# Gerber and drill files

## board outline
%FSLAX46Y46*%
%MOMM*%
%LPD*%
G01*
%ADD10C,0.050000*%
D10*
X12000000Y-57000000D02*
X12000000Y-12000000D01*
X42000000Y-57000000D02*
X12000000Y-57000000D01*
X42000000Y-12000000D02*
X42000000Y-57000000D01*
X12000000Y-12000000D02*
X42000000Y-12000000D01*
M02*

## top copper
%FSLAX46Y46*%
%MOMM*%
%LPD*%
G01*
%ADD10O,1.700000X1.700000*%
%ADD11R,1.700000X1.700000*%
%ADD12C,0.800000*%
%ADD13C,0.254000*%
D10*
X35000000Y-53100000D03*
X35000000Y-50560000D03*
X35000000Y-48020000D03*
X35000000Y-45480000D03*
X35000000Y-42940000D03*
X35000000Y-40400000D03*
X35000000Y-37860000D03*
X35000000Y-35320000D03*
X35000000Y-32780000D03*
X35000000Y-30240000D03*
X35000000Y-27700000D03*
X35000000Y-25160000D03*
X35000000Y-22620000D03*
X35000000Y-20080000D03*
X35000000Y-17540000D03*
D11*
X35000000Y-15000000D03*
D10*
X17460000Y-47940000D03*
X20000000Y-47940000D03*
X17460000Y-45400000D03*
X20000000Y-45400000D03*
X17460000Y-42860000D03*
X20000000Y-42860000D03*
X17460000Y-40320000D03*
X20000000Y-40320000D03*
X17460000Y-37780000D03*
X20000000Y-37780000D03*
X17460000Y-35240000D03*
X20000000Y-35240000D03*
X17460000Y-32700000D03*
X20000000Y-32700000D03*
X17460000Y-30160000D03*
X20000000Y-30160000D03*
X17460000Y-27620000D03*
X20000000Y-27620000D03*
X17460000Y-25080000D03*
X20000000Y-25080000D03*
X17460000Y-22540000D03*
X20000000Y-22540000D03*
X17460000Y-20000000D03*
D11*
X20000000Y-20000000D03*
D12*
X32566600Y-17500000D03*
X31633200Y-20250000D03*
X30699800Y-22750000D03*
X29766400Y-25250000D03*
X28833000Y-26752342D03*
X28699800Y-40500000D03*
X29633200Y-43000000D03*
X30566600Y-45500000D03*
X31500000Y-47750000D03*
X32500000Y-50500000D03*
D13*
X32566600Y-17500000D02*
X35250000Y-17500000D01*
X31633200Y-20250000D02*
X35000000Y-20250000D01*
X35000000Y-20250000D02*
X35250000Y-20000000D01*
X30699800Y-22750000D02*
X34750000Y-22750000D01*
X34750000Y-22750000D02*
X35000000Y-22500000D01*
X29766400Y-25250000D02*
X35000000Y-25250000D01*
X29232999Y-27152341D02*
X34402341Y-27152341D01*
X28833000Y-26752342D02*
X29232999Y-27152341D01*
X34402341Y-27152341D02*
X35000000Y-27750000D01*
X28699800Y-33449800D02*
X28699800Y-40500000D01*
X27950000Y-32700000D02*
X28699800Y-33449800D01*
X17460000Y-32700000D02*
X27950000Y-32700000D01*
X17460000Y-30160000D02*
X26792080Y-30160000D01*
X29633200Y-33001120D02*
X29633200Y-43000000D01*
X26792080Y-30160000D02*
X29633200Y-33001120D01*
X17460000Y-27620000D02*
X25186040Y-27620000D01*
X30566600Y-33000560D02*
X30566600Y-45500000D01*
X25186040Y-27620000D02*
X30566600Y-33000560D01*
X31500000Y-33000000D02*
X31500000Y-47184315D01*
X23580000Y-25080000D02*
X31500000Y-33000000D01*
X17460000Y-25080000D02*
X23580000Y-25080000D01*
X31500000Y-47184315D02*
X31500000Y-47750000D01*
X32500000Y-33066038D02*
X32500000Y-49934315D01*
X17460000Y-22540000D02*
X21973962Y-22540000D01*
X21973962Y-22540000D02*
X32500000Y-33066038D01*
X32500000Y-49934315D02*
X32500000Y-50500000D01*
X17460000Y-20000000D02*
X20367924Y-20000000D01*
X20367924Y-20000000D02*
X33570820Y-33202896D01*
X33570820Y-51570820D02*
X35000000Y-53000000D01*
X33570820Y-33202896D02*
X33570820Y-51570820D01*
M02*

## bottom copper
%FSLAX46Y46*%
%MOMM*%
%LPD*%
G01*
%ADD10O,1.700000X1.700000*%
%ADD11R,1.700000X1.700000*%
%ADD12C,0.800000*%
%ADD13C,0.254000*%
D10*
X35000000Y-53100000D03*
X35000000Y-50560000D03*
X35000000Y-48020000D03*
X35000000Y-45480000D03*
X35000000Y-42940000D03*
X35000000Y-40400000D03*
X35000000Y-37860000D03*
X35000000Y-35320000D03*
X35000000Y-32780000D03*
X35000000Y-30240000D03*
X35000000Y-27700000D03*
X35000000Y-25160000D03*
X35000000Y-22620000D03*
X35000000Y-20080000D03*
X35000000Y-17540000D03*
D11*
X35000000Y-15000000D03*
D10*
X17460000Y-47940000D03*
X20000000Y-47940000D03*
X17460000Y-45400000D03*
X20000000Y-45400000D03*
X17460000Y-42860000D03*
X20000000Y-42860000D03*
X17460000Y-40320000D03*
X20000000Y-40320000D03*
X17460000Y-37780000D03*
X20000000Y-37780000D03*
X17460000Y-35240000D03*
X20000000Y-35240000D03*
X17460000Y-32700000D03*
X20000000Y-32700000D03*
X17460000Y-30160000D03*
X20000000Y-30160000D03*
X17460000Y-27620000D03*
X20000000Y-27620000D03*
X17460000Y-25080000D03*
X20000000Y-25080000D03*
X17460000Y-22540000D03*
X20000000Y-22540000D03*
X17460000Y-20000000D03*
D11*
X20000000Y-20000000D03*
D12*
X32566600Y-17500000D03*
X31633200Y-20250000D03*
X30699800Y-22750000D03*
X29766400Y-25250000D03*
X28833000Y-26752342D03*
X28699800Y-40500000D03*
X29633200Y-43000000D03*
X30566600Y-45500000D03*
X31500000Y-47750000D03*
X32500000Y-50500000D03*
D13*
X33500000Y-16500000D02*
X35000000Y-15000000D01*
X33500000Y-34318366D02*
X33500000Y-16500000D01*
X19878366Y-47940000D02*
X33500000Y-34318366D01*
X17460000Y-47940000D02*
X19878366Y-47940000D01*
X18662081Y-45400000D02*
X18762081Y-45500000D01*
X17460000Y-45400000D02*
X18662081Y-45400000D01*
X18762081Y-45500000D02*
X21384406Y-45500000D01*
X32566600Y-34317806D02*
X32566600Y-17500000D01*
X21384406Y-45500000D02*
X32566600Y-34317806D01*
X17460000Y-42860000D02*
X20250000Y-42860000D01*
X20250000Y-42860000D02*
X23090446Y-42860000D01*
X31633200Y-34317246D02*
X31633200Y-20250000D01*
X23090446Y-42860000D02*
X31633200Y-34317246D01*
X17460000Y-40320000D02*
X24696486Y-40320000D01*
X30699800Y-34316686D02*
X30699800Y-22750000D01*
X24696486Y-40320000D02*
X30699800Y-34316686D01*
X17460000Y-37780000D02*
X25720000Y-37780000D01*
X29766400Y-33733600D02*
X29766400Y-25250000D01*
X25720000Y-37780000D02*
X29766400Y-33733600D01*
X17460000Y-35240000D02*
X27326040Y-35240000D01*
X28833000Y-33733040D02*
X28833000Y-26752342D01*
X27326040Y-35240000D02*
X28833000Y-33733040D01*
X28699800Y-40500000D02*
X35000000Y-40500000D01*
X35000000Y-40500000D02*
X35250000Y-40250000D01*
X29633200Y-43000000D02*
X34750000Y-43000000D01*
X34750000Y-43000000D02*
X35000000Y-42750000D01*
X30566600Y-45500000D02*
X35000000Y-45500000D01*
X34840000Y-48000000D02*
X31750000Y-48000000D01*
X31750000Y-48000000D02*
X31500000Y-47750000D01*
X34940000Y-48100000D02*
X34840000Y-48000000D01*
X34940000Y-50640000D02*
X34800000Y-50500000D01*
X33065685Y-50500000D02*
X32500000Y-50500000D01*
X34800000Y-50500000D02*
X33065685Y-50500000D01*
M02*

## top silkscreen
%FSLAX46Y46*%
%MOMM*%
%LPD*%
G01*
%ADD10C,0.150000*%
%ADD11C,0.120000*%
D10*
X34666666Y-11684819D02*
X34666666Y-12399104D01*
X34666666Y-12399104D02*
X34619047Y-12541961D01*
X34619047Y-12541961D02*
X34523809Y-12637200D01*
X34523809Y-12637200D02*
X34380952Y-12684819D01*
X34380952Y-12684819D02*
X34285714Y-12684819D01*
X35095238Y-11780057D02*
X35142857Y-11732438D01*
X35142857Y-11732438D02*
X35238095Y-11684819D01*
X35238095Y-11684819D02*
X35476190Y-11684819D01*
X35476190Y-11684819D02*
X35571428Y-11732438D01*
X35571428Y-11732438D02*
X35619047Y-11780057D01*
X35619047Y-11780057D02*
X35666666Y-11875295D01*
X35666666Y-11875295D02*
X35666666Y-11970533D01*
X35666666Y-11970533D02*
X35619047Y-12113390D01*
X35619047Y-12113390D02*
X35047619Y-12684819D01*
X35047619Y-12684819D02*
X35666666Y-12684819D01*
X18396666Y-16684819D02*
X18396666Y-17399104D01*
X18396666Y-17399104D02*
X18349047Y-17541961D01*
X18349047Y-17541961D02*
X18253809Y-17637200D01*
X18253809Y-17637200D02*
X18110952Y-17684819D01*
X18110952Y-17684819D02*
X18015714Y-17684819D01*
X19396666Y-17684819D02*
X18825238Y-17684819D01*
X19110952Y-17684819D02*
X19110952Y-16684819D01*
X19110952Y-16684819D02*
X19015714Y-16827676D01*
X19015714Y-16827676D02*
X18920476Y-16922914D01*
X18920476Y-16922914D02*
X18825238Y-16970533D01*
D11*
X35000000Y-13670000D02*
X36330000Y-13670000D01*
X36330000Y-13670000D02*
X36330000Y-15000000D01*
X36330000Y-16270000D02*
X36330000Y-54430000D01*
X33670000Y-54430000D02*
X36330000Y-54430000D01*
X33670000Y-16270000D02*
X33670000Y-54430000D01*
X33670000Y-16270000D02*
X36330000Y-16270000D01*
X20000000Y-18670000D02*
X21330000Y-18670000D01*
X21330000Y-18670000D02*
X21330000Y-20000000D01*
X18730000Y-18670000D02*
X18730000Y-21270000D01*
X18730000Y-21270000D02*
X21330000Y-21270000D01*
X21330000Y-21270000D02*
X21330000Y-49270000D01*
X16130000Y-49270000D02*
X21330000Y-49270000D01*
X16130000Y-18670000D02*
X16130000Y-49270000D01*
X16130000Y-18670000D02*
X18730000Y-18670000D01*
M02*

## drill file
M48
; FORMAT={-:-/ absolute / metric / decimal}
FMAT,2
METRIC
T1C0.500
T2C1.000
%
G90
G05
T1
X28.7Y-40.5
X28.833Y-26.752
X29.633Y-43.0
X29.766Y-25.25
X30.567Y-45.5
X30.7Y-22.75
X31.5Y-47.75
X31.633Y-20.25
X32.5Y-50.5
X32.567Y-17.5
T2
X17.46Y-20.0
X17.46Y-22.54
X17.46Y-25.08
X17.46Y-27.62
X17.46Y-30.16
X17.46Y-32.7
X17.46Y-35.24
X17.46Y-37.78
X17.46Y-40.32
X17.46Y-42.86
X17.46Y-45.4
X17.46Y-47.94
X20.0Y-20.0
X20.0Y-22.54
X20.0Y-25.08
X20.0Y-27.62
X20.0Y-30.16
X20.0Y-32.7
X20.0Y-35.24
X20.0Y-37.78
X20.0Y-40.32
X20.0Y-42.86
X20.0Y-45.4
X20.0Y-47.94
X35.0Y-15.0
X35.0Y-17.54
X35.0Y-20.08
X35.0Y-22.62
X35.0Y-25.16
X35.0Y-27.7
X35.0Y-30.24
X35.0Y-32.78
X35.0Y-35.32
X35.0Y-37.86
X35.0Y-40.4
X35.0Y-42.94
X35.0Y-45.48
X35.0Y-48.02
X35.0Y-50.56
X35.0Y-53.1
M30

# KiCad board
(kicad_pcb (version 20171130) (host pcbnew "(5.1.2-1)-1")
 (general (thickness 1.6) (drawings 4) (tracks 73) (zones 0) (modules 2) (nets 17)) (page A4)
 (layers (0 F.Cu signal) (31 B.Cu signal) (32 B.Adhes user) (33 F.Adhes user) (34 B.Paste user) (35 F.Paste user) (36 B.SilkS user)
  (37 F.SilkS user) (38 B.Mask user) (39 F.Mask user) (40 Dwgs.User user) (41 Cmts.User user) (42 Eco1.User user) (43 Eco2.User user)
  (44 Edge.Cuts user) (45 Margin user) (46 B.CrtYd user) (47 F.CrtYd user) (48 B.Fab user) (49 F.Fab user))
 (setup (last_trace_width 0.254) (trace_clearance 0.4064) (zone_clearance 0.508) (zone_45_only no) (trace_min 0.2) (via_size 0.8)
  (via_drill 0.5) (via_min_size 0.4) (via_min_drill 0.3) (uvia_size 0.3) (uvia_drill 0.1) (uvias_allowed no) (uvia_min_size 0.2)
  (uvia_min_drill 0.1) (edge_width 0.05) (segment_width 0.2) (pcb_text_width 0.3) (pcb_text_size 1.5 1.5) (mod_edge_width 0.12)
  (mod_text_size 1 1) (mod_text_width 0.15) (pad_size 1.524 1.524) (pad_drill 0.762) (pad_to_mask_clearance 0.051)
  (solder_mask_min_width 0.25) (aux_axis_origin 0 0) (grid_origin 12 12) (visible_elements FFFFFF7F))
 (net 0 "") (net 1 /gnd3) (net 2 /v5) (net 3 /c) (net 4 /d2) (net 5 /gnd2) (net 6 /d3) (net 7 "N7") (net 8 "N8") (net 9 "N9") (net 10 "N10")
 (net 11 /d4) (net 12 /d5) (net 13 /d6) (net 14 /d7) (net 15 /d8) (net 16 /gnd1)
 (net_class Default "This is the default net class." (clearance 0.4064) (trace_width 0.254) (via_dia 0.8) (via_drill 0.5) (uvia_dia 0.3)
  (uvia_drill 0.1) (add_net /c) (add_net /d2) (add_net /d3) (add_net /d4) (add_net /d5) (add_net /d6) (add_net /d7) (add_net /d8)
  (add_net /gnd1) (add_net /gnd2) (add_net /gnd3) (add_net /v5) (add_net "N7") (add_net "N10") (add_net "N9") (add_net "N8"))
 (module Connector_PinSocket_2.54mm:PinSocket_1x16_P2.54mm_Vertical (layer F.Cu) (at 35 15)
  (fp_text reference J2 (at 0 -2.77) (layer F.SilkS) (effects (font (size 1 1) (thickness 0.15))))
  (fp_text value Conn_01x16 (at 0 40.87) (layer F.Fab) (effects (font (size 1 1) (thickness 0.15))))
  (fp_line (start 0 -1.33) (end 1.33 -1.33) (layer F.SilkS) (width 0.12))
  (fp_line (start 1.33 -1.33) (end 1.33 0) (layer F.SilkS) (width 0.12))
  (fp_line (start 1.33 1.27) (end 1.33 39.43) (layer F.SilkS) (width 0.12))
  (fp_line (start -1.33 39.43) (end 1.33 39.43) (layer F.SilkS) (width 0.12))
  (fp_line (start -1.33 1.27) (end -1.33 39.43) (layer F.SilkS) (width 0.12))
  (fp_line (start -1.33 1.27) (end 1.33 1.27) (layer F.SilkS) (width 0.12))
  (pad 16 thru_hole oval (at 0 38.1) (size 1.7 1.7) (drill 1) (layers *.Cu *.Mask) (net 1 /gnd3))
  (pad 15 thru_hole oval (at 0 35.56) (size 1.7 1.7) (drill 1) (layers *.Cu *.Mask) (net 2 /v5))
  (pad 14 thru_hole oval (at 0 33.02) (size 1.7 1.7) (drill 1) (layers *.Cu *.Mask) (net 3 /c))
  (pad 13 thru_hole oval (at 0 30.48) (size 1.7 1.7) (drill 1) (layers *.Cu *.Mask) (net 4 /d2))
  (pad 12 thru_hole oval (at 0 27.94) (size 1.7 1.7) (drill 1) (layers *.Cu *.Mask) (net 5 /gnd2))
  (pad 11 thru_hole oval (at 0 25.4) (size 1.7 1.7) (drill 1) (layers *.Cu *.Mask) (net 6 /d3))
  (pad 10 thru_hole oval (at 0 22.86) (size 1.7 1.7) (drill 1) (layers *.Cu *.Mask) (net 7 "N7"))
  (pad 9 thru_hole oval (at 0 20.32) (size 1.7 1.7) (drill 1) (layers *.Cu *.Mask) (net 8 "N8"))
  (pad 8 thru_hole oval (at 0 17.78) (size 1.7 1.7) (drill 1) (layers *.Cu *.Mask) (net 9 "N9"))
  (pad 7 thru_hole oval (at 0 15.24) (size 1.7 1.7) (drill 1) (layers *.Cu *.Mask) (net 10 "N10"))
  (pad 6 thru_hole oval (at 0 12.7) (size 1.7 1.7) (drill 1) (layers *.Cu *.Mask) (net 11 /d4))
  (pad 5 thru_hole oval (at 0 10.16) (size 1.7 1.7) (drill 1) (layers *.Cu *.Mask) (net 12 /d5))
  (pad 4 thru_hole oval (at 0 7.62) (size 1.7 1.7) (drill 1) (layers *.Cu *.Mask) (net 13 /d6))
  (pad 3 thru_hole oval (at 0 5.08) (size 1.7 1.7) (drill 1) (layers *.Cu *.Mask) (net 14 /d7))
  (pad 2 thru_hole oval (at 0 2.54) (size 1.7 1.7) (drill 1) (layers *.Cu *.Mask) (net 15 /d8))
  (pad 1 thru_hole rect (at 0 0) (size 1.7 1.7) (drill 1) (layers *.Cu *.Mask) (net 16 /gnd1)))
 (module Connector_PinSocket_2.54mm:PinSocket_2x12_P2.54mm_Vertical (layer F.Cu) (at 20 20)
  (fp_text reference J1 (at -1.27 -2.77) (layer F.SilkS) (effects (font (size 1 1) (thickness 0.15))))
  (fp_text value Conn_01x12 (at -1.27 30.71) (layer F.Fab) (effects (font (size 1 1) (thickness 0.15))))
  (fp_line (start 0 -1.33) (end 1.33 -1.33) (layer F.SilkS) (width 0.12))
  (fp_line (start 1.33 -1.33) (end 1.33 0) (layer F.SilkS) (width 0.12))
  (fp_line (start -1.27 -1.33) (end -1.27 1.27) (layer F.SilkS) (width 0.12))
  (fp_line (start -1.27 1.27) (end 1.33 1.27) (layer F.SilkS) (width 0.12))
  (fp_line (start 1.33 1.27) (end 1.33 29.27) (layer F.SilkS) (width 0.12))
  (fp_line (start -3.87 29.27) (end 1.33 29.27) (layer F.SilkS) (width 0.12))
  (fp_line (start -3.87 -1.33) (end -3.87 29.27) (layer F.SilkS) (width 0.12))
  (fp_line (start -3.87 -1.33) (end -1.27 -1.33) (layer F.SilkS) (width 0.12))
  (pad 24 thru_hole oval (at -2.54 27.94) (size 1.7 1.7) (drill 1) (layers *.Cu *.Mask) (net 16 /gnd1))
  (pad 23 thru_hole oval (at 0 27.94) (size 1.7 1.7) (drill 1) (layers *.Cu *.Mask) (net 16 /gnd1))
  (pad 22 thru_hole oval (at -2.54 25.4) (size 1.7 1.7) (drill 1) (layers *.Cu *.Mask) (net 15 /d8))
  (pad 21 thru_hole oval (at 0 25.4) (size 1.7 1.7) (drill 1) (layers *.Cu *.Mask) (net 15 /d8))
  (pad 20 thru_hole oval (at -2.54 22.86) (size 1.7 1.7) (drill 1) (layers *.Cu *.Mask) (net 14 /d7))
  (pad 19 thru_hole oval (at 0 22.86) (size 1.7 1.7) (drill 1) (layers *.Cu *.Mask) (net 14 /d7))
  (pad 18 thru_hole oval (at -2.54 20.32) (size 1.7 1.7) (drill 1) (layers *.Cu *.Mask) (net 13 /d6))
  (pad 17 thru_hole oval (at 0 20.32) (size 1.7 1.7) (drill 1) (layers *.Cu *.Mask) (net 13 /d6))
  (pad 16 thru_hole oval (at -2.54 17.78) (size 1.7 1.7) (drill 1) (layers *.Cu *.Mask) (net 12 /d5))
  (pad 15 thru_hole oval (at 0 17.78) (size 1.7 1.7) (drill 1) (layers *.Cu *.Mask) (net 12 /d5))
  (pad 14 thru_hole oval (at -2.54 15.24) (size 1.7 1.7) (drill 1) (layers *.Cu *.Mask) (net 11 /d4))
  (pad 13 thru_hole oval (at 0 15.24) (size 1.7 1.7) (drill 1) (layers *.Cu *.Mask) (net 11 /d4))
  (pad 12 thru_hole oval (at -2.54 12.7) (size 1.7 1.7) (drill 1) (layers *.Cu *.Mask) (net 6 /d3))
  (pad 11 thru_hole oval (at 0 12.7) (size 1.7 1.7) (drill 1) (layers *.Cu *.Mask) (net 6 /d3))
  (pad 10 thru_hole oval (at -2.54 10.16) (size 1.7 1.7) (drill 1) (layers *.Cu *.Mask) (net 5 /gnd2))
  (pad 9 thru_hole oval (at 0 10.16) (size 1.7 1.7) (drill 1) (layers *.Cu *.Mask) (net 5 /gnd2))
  (pad 8 thru_hole oval (at -2.54 7.62) (size 1.7 1.7) (drill 1) (layers *.Cu *.Mask) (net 4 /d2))
  (pad 7 thru_hole oval (at 0 7.62) (size 1.7 1.7) (drill 1) (layers *.Cu *.Mask) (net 4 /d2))
  (pad 6 thru_hole oval (at -2.54 5.08) (size 1.7 1.7) (drill 1) (layers *.Cu *.Mask) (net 3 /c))
  (pad 5 thru_hole oval (at 0 5.08) (size 1.7 1.7) (drill 1) (layers *.Cu *.Mask) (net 3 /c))
  (pad 4 thru_hole oval (at -2.54 2.54) (size 1.7 1.7) (drill 1) (layers *.Cu *.Mask) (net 2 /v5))
  (pad 3 thru_hole oval (at 0 2.54) (size 1.7 1.7) (drill 1) (layers *.Cu *.Mask) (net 2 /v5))
  (pad 2 thru_hole oval (at -2.54 0) (size 1.7 1.7) (drill 1) (layers *.Cu *.Mask) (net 1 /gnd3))
  (pad 1 thru_hole rect (at 0 0) (size 1.7 1.7) (drill 1) (layers *.Cu *.Mask) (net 1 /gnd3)))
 (gr_line (start 12 57) (end 12 12) (layer Edge.Cuts) (width 0.05))
 (gr_line (start 42 57) (end 12 57) (layer Edge.Cuts) (width 0.05))
 (gr_line (start 42 12) (end 42 57) (layer Edge.Cuts) (width 0.05))
 (gr_line (start 12 12) (end 42 12) (layer Edge.Cuts) (width 0.05))
 (segment (start 33.5 16.5) (end 35 15) (width 0.254) (layer B.Cu) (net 16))
 (segment (start 33.5 34.318366) (end 33.5 16.5) (width 0.254) (layer B.Cu) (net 16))
 (segment (start 19.878366 47.94) (end 33.5 34.318366) (width 0.254) (layer B.Cu) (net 16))
 (segment (start 17.46 47.94) (end 19.878366 47.94) (width 0.254) (layer B.Cu) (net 16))
 (segment (start 18.662081 45.4) (end 18.762081 45.5) (width 0.254) (layer B.Cu) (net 15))
 (segment (start 17.46 45.4) (end 18.662081 45.4) (width 0.254) (layer B.Cu) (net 15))
 (segment (start 18.762081 45.5) (end 21.384406 45.5) (width 0.254) (layer B.Cu) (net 15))
 (via (at 32.5666 17.5) (size 0.8) (drill 0.5) (layers F.Cu B.Cu) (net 15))
 (segment (start 32.5666 34.317806) (end 32.5666 17.5) (width 0.254) (layer B.Cu) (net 15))
 (segment (start 21.384406 45.5) (end 32.5666 34.317806) (width 0.254) (layer B.Cu) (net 15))
 (segment (start 32.5666 17.5) (end 35.25 17.5) (width 0.254) (layer F.Cu) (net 15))
 (segment (start 17.46 42.86) (end 20.25 42.86) (width 0.254) (layer B.Cu) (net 14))
 (segment (start 20.25 42.86) (end 23.090446 42.86) (width 0.254) (layer B.Cu) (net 14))
 (via (at 31.6332 20.25) (size 0.8) (drill 0.5) (layers F.Cu B.Cu) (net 14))
 (segment (start 31.6332 34.317246) (end 31.6332 20.25) (width 0.254) (layer B.Cu) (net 14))
 (segment (start 23.090446 42.86) (end 31.6332 34.317246) (width 0.254) (layer B.Cu) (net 14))
 (segment (start 31.6332 20.25) (end 35 20.25) (width 0.254) (layer F.Cu) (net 14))
 (segment (start 35 20.25) (end 35.25 20) (width 0.254) (layer F.Cu) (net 14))
 (segment (start 17.46 40.32) (end 24.696486 40.32) (width 0.254) (layer B.Cu) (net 13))
 (via (at 30.6998 22.75) (size 0.8) (drill 0.5) (layers F.Cu B.Cu) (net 13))
 (segment (start 30.6998 34.316686) (end 30.6998 22.75) (width 0.254) (layer B.Cu) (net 13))
 (segment (start 24.696486 40.32) (end 30.6998 34.316686) (width 0.254) (layer B.Cu) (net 13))
 (segment (start 30.6998 22.75) (end 34.75 22.75) (width 0.254) (layer F.Cu) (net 13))
 (segment (start 34.75 22.75) (end 35 22.5) (width 0.254) (layer F.Cu) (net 13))
 (segment (start 17.46 37.78) (end 25.72 37.78) (width 0.254) (layer B.Cu) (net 12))
 (via (at 29.7664 25.25) (size 0.8) (drill 0.5) (layers F.Cu B.Cu) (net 12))
 (segment (start 29.7664 33.7336) (end 29.7664 25.25) (width 0.254) (layer B.Cu) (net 12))
 (segment (start 25.72 37.78) (end 29.7664 33.7336) (width 0.254) (layer B.Cu) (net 12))
 (segment (start 29.7664 25.25) (end 35 25.25) (width 0.254) (layer F.Cu) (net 12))
 (segment (start 17.46 35.24) (end 27.32604 35.24) (width 0.254) (layer B.Cu) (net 11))
 (via (at 28.833 26.752342) (size 0.8) (drill 0.5) (layers F.Cu B.Cu) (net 11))
 (segment (start 28.833 33.73304) (end 28.833 26.752342) (width 0.254) (layer B.Cu) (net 11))
 (segment (start 27.32604 35.24) (end 28.833 33.73304) (width 0.254) (layer B.Cu) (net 11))
 (segment (start 29.232999 27.152341) (end 34.402341 27.152341) (width 0.254) (layer F.Cu) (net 11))
 (segment (start 28.833 26.752342) (end 29.232999 27.152341) (width 0.254) (layer F.Cu) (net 11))
 (segment (start 34.402341 27.152341) (end 35 27.75) (width 0.254) (layer F.Cu) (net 11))
 (via (at 28.6998 40.5) (size 0.8) (drill 0.5) (layers F.Cu B.Cu) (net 6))
 (segment (start 28.6998 40.5) (end 35 40.5) (width 0.254) (layer B.Cu) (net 6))
 (segment (start 35 40.5) (end 35.25 40.25) (width 0.254) (layer B.Cu) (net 6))
 (segment (start 28.6998 33.4498) (end 28.6998 40.5) (width 0.254) (layer F.Cu) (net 6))
 (segment (start 27.95 32.7) (end 28.6998 33.4498) (width 0.254) (layer F.Cu) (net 6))
 (segment (start 17.46 32.7) (end 27.95 32.7) (width 0.254) (layer F.Cu) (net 6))
 (segment (start 17.46 30.16) (end 26.79208 30.16) (width 0.254) (layer F.Cu) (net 5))
 (segment (start 29.6332 33.00112) (end 29.6332 43) (width 0.254) (layer F.Cu) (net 5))
 (via (at 29.6332 43) (size 0.8) (drill 0.5) (layers F.Cu B.Cu) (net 5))
 (segment (start 26.79208 30.16) (end 29.6332 33.00112) (width 0.254) (layer F.Cu) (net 5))
 (segment (start 29.6332 43) (end 34.75 43) (width 0.254) (layer B.Cu) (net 5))
 (segment (start 34.75 43) (end 35 42.75) (width 0.254) (layer B.Cu) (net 5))
 (segment (start 17.46 27.62) (end 25.18604 27.62) (width 0.254) (layer F.Cu) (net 4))
 (via (at 30.5666 45.5) (size 0.8) (drill 0.5) (layers F.Cu B.Cu) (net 4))
 (segment (start 30.5666 33.00056) (end 30.5666 45.5) (width 0.254) (layer F.Cu) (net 4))
 (segment (start 25.18604 27.62) (end 30.5666 33.00056) (width 0.254) (layer F.Cu) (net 4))
 (segment (start 30.5666 45.5) (end 35 45.5) (width 0.254) (layer B.Cu) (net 4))
 (via (at 31.5 47.75) (size 0.8) (drill 0.5) (layers F.Cu B.Cu) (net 3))
 (segment (start 34.84 48) (end 31.75 48) (width 0.254) (layer B.Cu) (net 3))
 (segment (start 31.75 48) (end 31.5 47.75) (width 0.254) (layer B.Cu) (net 3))
 (segment (start 34.94 48.1) (end 34.84 48) (width 0.254) (layer B.Cu) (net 3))
 (segment (start 31.5 33) (end 31.5 47.184315) (width 0.254) (layer F.Cu) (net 3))
 (segment (start 23.58 25.08) (end 31.5 33) (width 0.254) (layer F.Cu) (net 3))
 (segment (start 17.46 25.08) (end 23.58 25.08) (width 0.254) (layer F.Cu) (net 3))
 (segment (start 31.5 47.184315) (end 31.5 47.75) (width 0.254) (layer F.Cu) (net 3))
 (segment (start 34.94 50.64) (end 34.8 50.5) (width 0.254) (layer B.Cu) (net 2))
 (via (at 32.5 50.5) (size 0.8) (drill 0.5) (layers F.Cu B.Cu) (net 2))
 (segment (start 33.065685 50.5) (end 32.5 50.5) (width 0.254) (layer B.Cu) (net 2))
 (segment (start 34.8 50.5) (end 33.065685 50.5) (width 0.254) (layer B.Cu) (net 2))
 (segment (start 32.5 33.066038) (end 32.5 49.934315) (width 0.254) (layer F.Cu) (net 2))
 (segment (start 17.46 22.54) (end 21.973962 22.54) (width 0.254) (layer F.Cu) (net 2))
 (segment (start 21.973962 22.54) (end 32.5 33.066038) (width 0.254) (layer F.Cu) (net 2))
 (segment (start 32.5 49.934315) (end 32.5 50.5) (width 0.254) (layer F.Cu) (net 2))
 (segment (start 17.46 20) (end 20.367924 20) (width 0.254) (layer F.Cu) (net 1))
 (segment (start 20.367924 20) (end 33.57082 33.202896) (width 0.254) (layer F.Cu) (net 1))
 (segment (start 33.57082 51.57082) (end 35 53) (width 0.254) (layer F.Cu) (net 1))
 (segment (start 33.57082 33.202896) (end 33.57082 51.57082) (width 0.254) (layer F.Cu) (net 1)))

